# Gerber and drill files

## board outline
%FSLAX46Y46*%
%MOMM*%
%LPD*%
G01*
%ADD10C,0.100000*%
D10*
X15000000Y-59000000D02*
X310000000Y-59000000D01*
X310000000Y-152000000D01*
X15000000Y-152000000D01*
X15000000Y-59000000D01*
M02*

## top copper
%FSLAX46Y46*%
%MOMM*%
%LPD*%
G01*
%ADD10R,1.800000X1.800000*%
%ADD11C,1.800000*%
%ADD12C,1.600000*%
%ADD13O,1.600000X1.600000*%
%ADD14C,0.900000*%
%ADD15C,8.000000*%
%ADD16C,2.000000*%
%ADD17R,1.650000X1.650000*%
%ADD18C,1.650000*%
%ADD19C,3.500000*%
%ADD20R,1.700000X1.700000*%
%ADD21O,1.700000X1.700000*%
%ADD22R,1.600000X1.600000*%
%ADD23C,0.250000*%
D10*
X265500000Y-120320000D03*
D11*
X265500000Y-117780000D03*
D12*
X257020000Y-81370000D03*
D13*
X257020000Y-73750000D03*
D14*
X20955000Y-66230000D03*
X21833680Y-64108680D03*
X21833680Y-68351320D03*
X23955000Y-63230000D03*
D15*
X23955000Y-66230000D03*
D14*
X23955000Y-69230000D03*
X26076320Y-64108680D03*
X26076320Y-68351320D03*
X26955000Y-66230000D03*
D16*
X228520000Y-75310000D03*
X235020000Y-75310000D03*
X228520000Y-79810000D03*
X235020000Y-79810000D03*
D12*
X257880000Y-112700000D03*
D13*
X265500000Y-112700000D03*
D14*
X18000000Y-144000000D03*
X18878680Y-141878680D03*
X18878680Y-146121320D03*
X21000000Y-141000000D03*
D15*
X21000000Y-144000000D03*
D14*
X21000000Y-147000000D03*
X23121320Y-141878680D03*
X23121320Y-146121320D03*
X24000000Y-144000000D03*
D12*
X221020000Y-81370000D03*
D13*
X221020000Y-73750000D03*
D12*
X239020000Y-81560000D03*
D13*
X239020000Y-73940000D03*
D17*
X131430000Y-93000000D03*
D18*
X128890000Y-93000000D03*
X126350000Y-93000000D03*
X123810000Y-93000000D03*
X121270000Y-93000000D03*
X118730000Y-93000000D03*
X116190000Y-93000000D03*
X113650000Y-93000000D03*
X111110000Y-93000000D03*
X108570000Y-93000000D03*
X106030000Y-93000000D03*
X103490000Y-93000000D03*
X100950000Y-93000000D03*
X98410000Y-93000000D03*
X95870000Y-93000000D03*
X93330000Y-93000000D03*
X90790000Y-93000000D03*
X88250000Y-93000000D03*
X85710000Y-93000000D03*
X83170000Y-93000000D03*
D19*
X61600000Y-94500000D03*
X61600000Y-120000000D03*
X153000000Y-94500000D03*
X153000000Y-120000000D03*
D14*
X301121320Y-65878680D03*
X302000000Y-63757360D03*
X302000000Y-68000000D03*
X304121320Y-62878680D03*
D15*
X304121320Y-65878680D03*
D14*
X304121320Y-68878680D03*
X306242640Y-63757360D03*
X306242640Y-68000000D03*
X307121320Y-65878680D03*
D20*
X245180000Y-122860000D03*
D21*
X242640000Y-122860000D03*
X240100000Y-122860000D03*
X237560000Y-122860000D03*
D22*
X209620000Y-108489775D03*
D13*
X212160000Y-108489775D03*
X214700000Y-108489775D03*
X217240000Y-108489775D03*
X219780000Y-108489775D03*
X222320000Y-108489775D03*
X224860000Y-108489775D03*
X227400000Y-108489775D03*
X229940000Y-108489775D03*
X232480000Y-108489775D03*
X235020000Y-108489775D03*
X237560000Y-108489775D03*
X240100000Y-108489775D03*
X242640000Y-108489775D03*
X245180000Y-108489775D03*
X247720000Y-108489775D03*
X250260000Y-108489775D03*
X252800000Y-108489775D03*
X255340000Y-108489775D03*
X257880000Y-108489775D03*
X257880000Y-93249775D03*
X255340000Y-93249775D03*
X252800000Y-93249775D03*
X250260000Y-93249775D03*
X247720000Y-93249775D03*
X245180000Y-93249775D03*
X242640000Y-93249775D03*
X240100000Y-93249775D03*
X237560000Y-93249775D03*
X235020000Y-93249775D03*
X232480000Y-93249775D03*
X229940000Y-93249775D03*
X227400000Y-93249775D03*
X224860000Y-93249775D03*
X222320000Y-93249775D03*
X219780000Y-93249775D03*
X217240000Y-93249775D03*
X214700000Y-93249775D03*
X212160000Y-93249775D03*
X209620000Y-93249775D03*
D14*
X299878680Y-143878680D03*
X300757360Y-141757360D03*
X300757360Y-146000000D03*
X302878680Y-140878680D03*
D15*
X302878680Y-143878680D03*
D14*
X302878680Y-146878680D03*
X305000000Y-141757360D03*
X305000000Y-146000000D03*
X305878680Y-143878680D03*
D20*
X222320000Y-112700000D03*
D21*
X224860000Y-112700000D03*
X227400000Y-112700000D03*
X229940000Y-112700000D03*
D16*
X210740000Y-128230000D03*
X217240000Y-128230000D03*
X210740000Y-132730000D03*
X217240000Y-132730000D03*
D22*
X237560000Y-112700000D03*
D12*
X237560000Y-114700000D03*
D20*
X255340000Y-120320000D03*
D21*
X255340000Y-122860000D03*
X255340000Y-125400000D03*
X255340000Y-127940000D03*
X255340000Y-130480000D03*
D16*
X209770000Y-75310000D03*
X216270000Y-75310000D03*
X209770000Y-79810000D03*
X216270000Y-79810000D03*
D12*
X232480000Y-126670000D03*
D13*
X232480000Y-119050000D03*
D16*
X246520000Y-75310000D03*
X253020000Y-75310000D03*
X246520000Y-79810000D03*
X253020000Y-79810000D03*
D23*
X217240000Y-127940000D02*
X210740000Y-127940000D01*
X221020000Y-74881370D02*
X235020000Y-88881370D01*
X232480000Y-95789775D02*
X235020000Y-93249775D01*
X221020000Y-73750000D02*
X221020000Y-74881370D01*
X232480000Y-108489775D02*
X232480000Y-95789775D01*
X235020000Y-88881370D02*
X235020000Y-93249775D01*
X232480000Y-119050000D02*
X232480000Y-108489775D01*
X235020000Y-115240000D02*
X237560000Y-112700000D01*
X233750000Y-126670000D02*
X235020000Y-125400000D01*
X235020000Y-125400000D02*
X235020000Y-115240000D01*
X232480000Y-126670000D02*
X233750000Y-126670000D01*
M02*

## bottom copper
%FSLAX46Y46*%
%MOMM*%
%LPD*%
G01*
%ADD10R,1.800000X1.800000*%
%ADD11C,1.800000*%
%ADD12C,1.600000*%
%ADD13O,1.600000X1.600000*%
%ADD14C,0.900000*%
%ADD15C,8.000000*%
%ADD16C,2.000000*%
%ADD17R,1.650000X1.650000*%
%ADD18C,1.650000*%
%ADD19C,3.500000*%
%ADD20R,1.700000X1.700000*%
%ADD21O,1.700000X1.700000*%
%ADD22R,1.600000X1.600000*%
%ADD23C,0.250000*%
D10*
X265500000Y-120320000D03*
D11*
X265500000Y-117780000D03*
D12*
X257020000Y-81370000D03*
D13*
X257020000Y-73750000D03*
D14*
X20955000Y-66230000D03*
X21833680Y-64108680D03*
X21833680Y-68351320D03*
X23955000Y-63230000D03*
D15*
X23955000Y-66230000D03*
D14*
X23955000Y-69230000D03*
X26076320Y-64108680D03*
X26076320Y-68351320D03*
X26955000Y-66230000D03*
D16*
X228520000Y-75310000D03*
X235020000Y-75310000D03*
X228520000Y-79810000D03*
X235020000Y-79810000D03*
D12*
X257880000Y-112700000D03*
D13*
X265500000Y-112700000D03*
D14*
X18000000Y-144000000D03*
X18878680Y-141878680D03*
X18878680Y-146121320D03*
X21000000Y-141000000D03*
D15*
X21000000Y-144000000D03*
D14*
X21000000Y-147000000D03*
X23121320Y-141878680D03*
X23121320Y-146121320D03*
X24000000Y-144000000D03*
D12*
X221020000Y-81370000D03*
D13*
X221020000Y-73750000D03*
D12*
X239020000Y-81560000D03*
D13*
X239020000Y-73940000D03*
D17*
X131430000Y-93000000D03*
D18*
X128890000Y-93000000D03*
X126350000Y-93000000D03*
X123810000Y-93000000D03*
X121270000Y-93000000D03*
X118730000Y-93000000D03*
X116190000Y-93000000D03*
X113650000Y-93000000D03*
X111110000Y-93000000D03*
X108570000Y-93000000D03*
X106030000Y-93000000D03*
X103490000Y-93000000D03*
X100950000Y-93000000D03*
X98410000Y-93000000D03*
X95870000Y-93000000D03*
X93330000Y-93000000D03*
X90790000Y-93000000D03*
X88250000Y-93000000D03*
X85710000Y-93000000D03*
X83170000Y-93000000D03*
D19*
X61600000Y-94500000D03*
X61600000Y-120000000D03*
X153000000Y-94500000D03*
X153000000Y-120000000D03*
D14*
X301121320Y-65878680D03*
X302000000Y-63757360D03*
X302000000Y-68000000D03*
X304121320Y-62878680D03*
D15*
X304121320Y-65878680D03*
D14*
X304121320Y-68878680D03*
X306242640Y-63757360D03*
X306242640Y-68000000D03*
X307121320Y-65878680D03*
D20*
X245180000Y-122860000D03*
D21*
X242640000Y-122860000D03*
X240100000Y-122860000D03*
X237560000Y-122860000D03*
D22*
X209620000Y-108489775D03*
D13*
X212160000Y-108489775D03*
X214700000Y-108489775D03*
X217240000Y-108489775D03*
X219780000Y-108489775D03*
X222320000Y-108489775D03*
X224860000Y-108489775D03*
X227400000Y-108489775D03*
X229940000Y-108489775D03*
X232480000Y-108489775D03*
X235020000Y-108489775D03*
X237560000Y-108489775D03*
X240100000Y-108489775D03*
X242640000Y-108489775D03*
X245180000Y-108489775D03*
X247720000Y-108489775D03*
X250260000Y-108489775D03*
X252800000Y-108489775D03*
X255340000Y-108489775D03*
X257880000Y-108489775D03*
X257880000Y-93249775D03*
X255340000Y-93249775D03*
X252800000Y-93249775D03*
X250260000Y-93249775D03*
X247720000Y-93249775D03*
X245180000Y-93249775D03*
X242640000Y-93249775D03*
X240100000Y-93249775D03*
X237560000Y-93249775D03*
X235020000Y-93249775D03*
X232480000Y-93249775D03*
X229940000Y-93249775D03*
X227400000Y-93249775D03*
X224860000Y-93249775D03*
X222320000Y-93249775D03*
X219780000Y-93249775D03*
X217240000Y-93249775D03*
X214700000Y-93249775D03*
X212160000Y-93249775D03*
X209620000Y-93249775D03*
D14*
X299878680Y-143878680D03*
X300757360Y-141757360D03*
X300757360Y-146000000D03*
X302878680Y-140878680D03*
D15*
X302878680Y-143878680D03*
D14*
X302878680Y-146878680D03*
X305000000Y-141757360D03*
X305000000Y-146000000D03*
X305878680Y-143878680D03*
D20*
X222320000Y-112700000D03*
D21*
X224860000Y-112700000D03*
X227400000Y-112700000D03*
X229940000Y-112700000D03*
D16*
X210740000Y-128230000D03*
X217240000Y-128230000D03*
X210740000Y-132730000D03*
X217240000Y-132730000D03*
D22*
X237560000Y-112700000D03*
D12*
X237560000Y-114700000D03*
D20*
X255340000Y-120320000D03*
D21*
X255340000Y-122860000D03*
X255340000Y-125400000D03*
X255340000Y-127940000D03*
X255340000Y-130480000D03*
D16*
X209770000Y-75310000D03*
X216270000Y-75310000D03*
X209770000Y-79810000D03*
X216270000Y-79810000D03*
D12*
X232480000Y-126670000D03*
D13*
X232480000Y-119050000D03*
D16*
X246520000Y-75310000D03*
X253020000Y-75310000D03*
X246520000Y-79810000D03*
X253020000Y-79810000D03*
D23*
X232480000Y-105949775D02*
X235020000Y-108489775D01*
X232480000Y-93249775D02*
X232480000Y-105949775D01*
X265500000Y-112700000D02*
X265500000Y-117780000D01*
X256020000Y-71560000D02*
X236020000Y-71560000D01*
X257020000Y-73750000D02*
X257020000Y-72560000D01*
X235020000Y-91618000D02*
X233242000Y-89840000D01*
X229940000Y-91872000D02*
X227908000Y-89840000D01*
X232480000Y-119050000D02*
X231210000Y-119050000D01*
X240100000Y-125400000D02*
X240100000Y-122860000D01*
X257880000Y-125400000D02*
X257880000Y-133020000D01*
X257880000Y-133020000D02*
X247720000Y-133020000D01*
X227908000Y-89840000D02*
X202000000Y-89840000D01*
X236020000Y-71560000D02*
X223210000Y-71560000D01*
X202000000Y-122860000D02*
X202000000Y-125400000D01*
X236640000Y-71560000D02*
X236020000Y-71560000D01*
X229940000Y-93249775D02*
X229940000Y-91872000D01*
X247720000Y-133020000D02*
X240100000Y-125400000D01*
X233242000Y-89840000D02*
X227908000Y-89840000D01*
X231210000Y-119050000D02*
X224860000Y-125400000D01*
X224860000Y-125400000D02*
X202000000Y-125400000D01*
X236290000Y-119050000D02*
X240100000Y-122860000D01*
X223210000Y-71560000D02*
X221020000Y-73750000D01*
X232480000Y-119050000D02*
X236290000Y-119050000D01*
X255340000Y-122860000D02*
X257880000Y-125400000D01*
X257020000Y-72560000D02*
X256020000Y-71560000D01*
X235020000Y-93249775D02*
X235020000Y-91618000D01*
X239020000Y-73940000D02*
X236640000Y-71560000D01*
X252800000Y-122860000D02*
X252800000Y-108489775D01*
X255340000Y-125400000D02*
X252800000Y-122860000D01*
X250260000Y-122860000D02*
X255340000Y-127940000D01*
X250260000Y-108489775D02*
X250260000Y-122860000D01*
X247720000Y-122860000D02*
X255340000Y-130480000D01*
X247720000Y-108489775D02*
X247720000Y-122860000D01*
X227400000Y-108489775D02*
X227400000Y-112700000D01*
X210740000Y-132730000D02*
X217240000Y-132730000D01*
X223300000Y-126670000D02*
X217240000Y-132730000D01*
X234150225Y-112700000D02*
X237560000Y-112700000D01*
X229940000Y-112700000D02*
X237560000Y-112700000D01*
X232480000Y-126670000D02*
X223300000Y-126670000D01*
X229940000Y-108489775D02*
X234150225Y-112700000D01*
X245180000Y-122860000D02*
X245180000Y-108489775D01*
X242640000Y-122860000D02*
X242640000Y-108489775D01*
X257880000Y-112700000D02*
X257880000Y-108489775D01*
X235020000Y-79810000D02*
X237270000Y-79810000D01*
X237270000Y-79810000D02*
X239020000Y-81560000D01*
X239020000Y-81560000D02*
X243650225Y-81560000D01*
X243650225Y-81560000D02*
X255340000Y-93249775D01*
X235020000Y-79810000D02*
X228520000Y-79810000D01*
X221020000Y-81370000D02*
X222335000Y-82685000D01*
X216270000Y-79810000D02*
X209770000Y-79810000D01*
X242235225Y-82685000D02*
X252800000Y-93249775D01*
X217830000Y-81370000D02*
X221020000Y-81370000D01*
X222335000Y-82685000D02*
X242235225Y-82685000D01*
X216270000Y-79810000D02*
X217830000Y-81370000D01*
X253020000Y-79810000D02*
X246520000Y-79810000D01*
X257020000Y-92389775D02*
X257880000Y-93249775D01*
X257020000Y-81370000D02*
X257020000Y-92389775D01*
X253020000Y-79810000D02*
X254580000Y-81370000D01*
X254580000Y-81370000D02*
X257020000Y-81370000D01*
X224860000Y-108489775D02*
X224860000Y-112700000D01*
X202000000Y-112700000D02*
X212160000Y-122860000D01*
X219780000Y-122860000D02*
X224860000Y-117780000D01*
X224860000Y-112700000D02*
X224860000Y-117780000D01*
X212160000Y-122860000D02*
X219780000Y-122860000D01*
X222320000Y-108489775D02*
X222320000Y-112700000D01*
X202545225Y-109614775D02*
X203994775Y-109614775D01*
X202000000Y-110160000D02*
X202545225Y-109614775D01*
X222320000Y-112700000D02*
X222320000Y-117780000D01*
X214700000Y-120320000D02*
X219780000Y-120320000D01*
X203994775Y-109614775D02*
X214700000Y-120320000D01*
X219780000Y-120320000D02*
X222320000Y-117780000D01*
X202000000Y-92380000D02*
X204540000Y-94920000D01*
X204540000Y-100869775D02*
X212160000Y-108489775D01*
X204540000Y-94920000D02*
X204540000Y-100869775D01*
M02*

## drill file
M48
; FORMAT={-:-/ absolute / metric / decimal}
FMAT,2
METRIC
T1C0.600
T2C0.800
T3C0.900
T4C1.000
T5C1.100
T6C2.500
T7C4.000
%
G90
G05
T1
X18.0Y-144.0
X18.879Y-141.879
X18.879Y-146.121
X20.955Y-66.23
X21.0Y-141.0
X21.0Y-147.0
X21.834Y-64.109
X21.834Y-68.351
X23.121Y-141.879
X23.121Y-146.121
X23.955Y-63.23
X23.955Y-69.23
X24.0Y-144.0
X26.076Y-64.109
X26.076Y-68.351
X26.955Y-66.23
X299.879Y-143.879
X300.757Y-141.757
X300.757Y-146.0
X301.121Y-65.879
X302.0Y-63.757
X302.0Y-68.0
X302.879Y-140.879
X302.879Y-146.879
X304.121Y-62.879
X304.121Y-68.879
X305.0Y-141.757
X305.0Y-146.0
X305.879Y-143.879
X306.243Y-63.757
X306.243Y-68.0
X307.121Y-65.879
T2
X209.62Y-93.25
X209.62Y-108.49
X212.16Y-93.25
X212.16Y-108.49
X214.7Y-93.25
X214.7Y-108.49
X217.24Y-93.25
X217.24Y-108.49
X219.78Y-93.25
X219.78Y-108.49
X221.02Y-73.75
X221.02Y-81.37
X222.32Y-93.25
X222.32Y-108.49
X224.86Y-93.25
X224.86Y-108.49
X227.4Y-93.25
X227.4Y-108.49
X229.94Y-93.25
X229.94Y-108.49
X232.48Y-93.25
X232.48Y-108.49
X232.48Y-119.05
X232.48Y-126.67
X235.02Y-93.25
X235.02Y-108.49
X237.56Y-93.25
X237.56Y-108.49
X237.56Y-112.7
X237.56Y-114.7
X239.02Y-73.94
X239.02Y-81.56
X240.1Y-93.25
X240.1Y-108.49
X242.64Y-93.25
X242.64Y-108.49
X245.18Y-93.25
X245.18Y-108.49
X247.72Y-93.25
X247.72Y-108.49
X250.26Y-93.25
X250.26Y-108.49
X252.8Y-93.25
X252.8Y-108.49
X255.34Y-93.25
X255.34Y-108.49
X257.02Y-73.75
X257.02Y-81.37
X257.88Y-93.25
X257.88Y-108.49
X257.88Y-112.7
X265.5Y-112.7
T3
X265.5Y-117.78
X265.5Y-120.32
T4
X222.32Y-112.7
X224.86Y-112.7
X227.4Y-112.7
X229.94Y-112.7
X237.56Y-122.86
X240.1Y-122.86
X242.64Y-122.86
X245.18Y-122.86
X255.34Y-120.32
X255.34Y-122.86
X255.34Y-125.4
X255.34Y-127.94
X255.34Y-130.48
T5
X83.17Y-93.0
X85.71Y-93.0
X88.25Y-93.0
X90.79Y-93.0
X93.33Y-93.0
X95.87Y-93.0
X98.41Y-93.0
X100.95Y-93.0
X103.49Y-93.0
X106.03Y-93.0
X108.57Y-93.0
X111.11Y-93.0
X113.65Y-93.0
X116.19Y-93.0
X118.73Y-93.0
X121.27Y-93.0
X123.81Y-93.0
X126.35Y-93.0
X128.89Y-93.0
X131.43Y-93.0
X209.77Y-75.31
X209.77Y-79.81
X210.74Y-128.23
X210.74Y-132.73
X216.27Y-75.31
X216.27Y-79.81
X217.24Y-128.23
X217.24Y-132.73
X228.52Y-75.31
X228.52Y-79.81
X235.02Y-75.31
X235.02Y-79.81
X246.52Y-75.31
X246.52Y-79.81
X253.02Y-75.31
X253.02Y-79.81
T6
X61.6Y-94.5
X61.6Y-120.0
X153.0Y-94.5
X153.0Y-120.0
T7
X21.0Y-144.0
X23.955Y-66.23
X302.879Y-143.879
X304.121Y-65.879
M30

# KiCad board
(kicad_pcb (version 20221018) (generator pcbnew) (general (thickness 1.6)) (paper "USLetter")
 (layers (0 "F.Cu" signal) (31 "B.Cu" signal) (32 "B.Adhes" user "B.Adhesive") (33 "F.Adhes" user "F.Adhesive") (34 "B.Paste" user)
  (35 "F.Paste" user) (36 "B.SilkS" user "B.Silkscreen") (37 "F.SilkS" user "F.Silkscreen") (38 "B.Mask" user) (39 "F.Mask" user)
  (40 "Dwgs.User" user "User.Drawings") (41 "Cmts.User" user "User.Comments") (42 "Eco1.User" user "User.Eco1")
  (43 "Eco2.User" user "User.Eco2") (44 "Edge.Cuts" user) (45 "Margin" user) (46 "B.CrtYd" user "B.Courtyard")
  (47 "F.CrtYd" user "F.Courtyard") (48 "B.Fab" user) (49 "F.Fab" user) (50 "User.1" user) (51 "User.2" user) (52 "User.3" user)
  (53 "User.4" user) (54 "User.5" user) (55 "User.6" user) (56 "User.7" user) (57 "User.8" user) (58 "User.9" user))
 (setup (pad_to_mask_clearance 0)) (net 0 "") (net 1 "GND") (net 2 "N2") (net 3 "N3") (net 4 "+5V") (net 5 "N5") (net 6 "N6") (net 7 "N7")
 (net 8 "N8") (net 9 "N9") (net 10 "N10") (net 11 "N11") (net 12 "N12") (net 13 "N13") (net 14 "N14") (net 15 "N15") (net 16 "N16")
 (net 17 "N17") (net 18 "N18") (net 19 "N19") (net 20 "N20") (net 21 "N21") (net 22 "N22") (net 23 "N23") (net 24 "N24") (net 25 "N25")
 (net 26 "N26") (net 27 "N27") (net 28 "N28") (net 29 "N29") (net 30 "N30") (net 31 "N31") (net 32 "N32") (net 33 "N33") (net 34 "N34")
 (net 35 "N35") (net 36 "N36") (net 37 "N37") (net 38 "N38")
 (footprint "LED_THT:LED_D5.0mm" (layer "F.Cu") (at 265.5 120.32 90)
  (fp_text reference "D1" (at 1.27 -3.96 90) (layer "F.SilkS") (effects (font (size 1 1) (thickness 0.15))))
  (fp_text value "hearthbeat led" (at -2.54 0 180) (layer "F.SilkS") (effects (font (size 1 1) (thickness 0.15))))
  (pad "1" thru_hole rect (at 0 0 90) (size 1.8 1.8) (drill 0.9) (layers "*.Cu" "*.Mask") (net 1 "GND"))
  (pad "2" thru_hole circle (at 2.54 0 90) (size 1.8 1.8) (drill 0.9) (layers "*.Cu" "*.Mask") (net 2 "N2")))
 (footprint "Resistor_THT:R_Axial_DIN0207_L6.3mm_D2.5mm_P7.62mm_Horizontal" (layer "F.Cu") (at 257.02 81.37 90)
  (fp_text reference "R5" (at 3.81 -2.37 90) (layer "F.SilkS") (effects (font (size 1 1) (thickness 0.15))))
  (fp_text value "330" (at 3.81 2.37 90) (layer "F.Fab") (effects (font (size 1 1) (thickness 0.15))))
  (pad "1" thru_hole circle (at 0 0 90) (size 1.6 1.6) (drill 0.8) (layers "*.Cu" "*.Mask") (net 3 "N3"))
  (pad "2" thru_hole oval (at 7.62 0 90) (size 1.6 1.6) (drill 0.8) (layers "*.Cu" "*.Mask") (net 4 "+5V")))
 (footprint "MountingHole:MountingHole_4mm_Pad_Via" (layer "F.Cu") (at 23.955 66.23)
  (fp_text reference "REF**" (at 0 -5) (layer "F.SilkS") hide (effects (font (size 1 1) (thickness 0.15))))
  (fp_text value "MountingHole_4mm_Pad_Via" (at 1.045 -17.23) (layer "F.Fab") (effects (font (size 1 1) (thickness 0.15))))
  (pad "1" thru_hole circle (at -3 0) (size 0.9 0.9) (drill 0.6) (layers "*.Cu" "*.Mask"))
  (pad "1" thru_hole circle (at -2.12132 -2.12132) (size 0.9 0.9) (drill 0.6) (layers "*.Cu" "*.Mask"))
  (pad "1" thru_hole circle (at -2.12132 2.12132) (size 0.9 0.9) (drill 0.6) (layers "*.Cu" "*.Mask"))
  (pad "1" thru_hole circle (at 0 -3) (size 0.9 0.9) (drill 0.6) (layers "*.Cu" "*.Mask"))
  (pad "1" thru_hole circle (at 0 0) (size 8 8) (drill 4) (layers "*.Cu" "*.Mask"))
  (pad "1" thru_hole circle (at 0 3) (size 0.9 0.9) (drill 0.6) (layers "*.Cu" "*.Mask"))
  (pad "1" thru_hole circle (at 2.12132 -2.12132) (size 0.9 0.9) (drill 0.6) (layers "*.Cu" "*.Mask"))
  (pad "1" thru_hole circle (at 2.12132 2.12132) (size 0.9 0.9) (drill 0.6) (layers "*.Cu" "*.Mask"))
  (pad "1" thru_hole circle (at 3 0) (size 0.9 0.9) (drill 0.6) (layers "*.Cu" "*.Mask")))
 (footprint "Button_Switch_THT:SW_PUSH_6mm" (layer "F.Cu") (at 228.52 75.31)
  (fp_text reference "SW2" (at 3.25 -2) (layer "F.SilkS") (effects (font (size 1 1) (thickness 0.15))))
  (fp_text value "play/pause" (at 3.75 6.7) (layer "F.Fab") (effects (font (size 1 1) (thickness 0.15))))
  (pad "1" thru_hole circle (at 0 0 90) (size 2 2) (drill 1.1) (layers "*.Cu" "*.Mask") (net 1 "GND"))
  (pad "1" thru_hole circle (at 6.5 0 90) (size 2 2) (drill 1.1) (layers "*.Cu" "*.Mask") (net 1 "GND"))
  (pad "2" thru_hole circle (at 0 4.5 90) (size 2 2) (drill 1.1) (layers "*.Cu" "*.Mask") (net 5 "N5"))
  (pad "2" thru_hole circle (at 6.5 4.5 90) (size 2 2) (drill 1.1) (layers "*.Cu" "*.Mask") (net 5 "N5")))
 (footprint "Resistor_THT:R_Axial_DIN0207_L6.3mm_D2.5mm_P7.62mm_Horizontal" (layer "F.Cu") (at 257.88 112.7)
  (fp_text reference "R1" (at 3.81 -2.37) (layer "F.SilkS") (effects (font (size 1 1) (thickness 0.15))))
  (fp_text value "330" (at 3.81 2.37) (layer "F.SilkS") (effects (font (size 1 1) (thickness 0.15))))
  (pad "1" thru_hole circle (at 0 0) (size 1.6 1.6) (drill 0.8) (layers "*.Cu" "*.Mask") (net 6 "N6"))
  (pad "2" thru_hole oval (at 7.62 0) (size 1.6 1.6) (drill 0.8) (layers "*.Cu" "*.Mask") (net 2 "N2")))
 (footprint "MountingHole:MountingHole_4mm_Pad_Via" (layer "F.Cu") (at 21 144)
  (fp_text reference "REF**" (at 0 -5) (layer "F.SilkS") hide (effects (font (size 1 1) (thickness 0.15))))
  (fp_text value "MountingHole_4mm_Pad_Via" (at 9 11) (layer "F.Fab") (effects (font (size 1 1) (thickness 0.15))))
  (pad "1" thru_hole circle (at -3 0) (size 0.9 0.9) (drill 0.6) (layers "*.Cu" "*.Mask"))
  (pad "1" thru_hole circle (at -2.12132 -2.12132) (size 0.9 0.9) (drill 0.6) (layers "*.Cu" "*.Mask"))
  (pad "1" thru_hole circle (at -2.12132 2.12132) (size 0.9 0.9) (drill 0.6) (layers "*.Cu" "*.Mask"))
  (pad "1" thru_hole circle (at 0 -3) (size 0.9 0.9) (drill 0.6) (layers "*.Cu" "*.Mask"))
  (pad "1" thru_hole circle (at 0 0) (size 8 8) (drill 4) (layers "*.Cu" "*.Mask"))
  (pad "1" thru_hole circle (at 0 3) (size 0.9 0.9) (drill 0.6) (layers "*.Cu" "*.Mask"))
  (pad "1" thru_hole circle (at 2.12132 -2.12132) (size 0.9 0.9) (drill 0.6) (layers "*.Cu" "*.Mask"))
  (pad "1" thru_hole circle (at 2.12132 2.12132) (size 0.9 0.9) (drill 0.6) (layers "*.Cu" "*.Mask"))
  (pad "1" thru_hole circle (at 3 0) (size 0.9 0.9) (drill 0.6) (layers "*.Cu" "*.Mask")))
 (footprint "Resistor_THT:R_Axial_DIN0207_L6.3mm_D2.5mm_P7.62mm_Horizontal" (layer "F.Cu") (at 221.02 81.37 90)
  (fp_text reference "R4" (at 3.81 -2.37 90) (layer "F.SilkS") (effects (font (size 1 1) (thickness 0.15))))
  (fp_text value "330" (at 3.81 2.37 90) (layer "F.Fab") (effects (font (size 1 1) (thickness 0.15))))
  (pad "1" thru_hole circle (at 0 0 90) (size 1.6 1.6) (drill 0.8) (layers "*.Cu" "*.Mask") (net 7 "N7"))
  (pad "2" thru_hole oval (at 7.62 0 90) (size 1.6 1.6) (drill 0.8) (layers "*.Cu" "*.Mask") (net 4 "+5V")))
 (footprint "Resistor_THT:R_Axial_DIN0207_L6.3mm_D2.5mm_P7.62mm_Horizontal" (layer "F.Cu") (at 239.02 81.56 90)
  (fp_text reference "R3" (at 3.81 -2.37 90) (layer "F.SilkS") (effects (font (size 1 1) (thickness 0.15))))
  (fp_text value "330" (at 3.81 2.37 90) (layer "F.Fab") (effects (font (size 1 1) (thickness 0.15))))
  (pad "1" thru_hole circle (at 0 0 90) (size 1.6 1.6) (drill 0.8) (layers "*.Cu" "*.Mask") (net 5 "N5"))
  (pad "2" thru_hole oval (at 7.62 0 90) (size 1.6 1.6) (drill 0.8) (layers "*.Cu" "*.Mask") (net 4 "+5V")))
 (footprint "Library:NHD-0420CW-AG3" (layer "F.Cu") (at 107.3 107.25)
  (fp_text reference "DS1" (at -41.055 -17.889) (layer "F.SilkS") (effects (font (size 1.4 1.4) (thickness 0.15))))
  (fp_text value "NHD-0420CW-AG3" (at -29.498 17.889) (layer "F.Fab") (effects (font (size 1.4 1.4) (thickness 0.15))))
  (pad "1" thru_hole rect (at 24.13 -14.25) (size 1.65 1.65) (drill 1.1) (layers "*.Cu" "*.Mask") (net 1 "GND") (solder_mask_margin 0.102))
  (pad "2" thru_hole circle (at 21.59 -14.25) (size 1.65 1.65) (drill 1.1) (layers "*.Cu" "*.Mask") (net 4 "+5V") (solder_mask_margin 0.102))
  (pad "3" thru_hole circle (at 19.05 -14.25) (size 1.65 1.65) (drill 1.1) (layers "*.Cu" "*.Mask") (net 4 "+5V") (solder_mask_margin 0.102))
  (pad "4" thru_hole circle (at 16.51 -14.25) (size 1.65 1.65) (drill 1.1) (layers "*.Cu" "*.Mask") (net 1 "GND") (solder_mask_margin 0.102))
  (pad "5" thru_hole circle (at 13.97 -14.25) (size 1.65 1.65) (drill 1.1) (layers "*.Cu" "*.Mask") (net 1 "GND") (solder_mask_margin 0.102))
  (pad "6" thru_hole circle (at 11.43 -14.25) (size 1.65 1.65) (drill 1.1) (layers "*.Cu" "*.Mask") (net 1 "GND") (solder_mask_margin 0.102))
  (pad "7" thru_hole circle (at 8.89 -14.25) (size 1.65 1.65) (drill 1.1) (layers "*.Cu" "*.Mask") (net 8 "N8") (solder_mask_margin 0.102))
  (pad "8" thru_hole circle (at 6.35 -14.25) (size 1.65 1.65) (drill 1.1) (layers "*.Cu" "*.Mask") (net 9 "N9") (solder_mask_margin 0.102))
  (pad "9" thru_hole circle (at 3.81 -14.25) (size 1.65 1.65) (drill 1.1) (layers "*.Cu" "*.Mask") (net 1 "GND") (solder_mask_margin 0.102))
  (pad "10" thru_hole circle (at 1.27 -14.25) (size 1.65 1.65) (drill 1.1) (layers "*.Cu" "*.Mask") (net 1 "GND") (solder_mask_margin 0.102))
  (pad "11" thru_hole circle (at -1.27 -14.25) (size 1.65 1.65) (drill 1.1) (layers "*.Cu" "*.Mask") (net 1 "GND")
   (solder_mask_margin 0.102))
  (pad "12" thru_hole circle (at -3.81 -14.25) (size 1.65 1.65) (drill 1.1) (layers "*.Cu" "*.Mask") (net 1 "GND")
   (solder_mask_margin 0.102))
  (pad "13" thru_hole circle (at -6.35 -14.25) (size 1.65 1.65) (drill 1.1) (layers "*.Cu" "*.Mask") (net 1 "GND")
   (solder_mask_margin 0.102))
  (pad "14" thru_hole circle (at -8.89 -14.25) (size 1.65 1.65) (drill 1.1) (layers "*.Cu" "*.Mask") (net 1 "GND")
   (solder_mask_margin 0.102))
  (pad "15" thru_hole circle (at -11.43 -14.25) (size 1.65 1.65) (drill 1.1) (layers "*.Cu" "*.Mask") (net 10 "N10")
   (solder_mask_margin 0.102))
  (pad "16" thru_hole circle (at -13.97 -14.25) (size 1.65 1.65) (drill 1.1) (layers "*.Cu" "*.Mask") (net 4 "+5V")
   (solder_mask_margin 0.102))
  (pad "17" thru_hole circle (at -16.51 -14.25) (size 1.65 1.65) (drill 1.1) (layers "*.Cu" "*.Mask") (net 1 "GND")
   (solder_mask_margin 0.102))
  (pad "18" thru_hole circle (at -19.05 -14.25) (size 1.65 1.65) (drill 1.1) (layers "*.Cu" "*.Mask") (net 1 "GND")
   (solder_mask_margin 0.102))
  (pad "19" thru_hole circle (at -21.59 -14.25) (size 1.65 1.65) (drill 1.1) (layers "*.Cu" "*.Mask") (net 1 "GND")
   (solder_mask_margin 0.102))
  (pad "20" thru_hole circle (at -24.13 -14.25) (size 1.65 1.65) (drill 1.1) (layers "*.Cu" "*.Mask") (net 1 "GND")
   (solder_mask_margin 0.102))
  (pad "P1" thru_hole circle (at -45.7 -12.75) (size 3.5 3.5) (drill 2.5) (layers "*.Cu" "*.Mask") (solder_mask_margin 0.102))
  (pad "P2" thru_hole circle (at -45.7 12.75) (size 3.5 3.5) (drill 2.5) (layers "*.Cu" "*.Mask") (solder_mask_margin 0.102))
  (pad "P3" thru_hole circle (at 45.7 -12.75) (size 3.5 3.5) (drill 2.5) (layers "*.Cu" "*.Mask") (solder_mask_margin 0.102))
  (pad "P4" thru_hole circle (at 45.7 12.75) (size 3.5 3.5) (drill 2.5) (layers "*.Cu" "*.Mask") (solder_mask_margin 0.102)))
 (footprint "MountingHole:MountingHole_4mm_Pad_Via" (layer "F.Cu") (at 304.12132 65.87868)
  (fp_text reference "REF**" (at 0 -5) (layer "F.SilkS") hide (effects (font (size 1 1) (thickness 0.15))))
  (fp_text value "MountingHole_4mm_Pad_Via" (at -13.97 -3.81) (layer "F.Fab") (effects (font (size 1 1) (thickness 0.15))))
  (pad "1" thru_hole circle (at -3 0) (size 0.9 0.9) (drill 0.6) (layers "*.Cu" "*.Mask"))
  (pad "1" thru_hole circle (at -2.12132 -2.12132) (size 0.9 0.9) (drill 0.6) (layers "*.Cu" "*.Mask"))
  (pad "1" thru_hole circle (at -2.12132 2.12132) (size 0.9 0.9) (drill 0.6) (layers "*.Cu" "*.Mask"))
  (pad "1" thru_hole circle (at 0 -3) (size 0.9 0.9) (drill 0.6) (layers "*.Cu" "*.Mask"))
  (pad "1" thru_hole circle (at 0 0) (size 8 8) (drill 4) (layers "*.Cu" "*.Mask"))
  (pad "1" thru_hole circle (at 0 3) (size 0.9 0.9) (drill 0.6) (layers "*.Cu" "*.Mask"))
  (pad "1" thru_hole circle (at 2.12132 -2.12132) (size 0.9 0.9) (drill 0.6) (layers "*.Cu" "*.Mask"))
  (pad "1" thru_hole circle (at 2.12132 2.12132) (size 0.9 0.9) (drill 0.6) (layers "*.Cu" "*.Mask"))
  (pad "1" thru_hole circle (at 3 0) (size 0.9 0.9) (drill 0.6) (layers "*.Cu" "*.Mask")))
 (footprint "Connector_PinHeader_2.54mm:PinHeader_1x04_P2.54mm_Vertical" (layer "F.Cu") (at 245.18 122.86 -90)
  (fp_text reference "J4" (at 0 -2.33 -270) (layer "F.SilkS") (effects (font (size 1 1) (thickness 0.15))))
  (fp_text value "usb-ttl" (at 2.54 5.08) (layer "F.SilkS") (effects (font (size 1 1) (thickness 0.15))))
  (pad "1" thru_hole rect (at 0 0 270) (size 1.7 1.7) (drill 1) (layers "*.Cu" "*.Mask") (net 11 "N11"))
  (pad "2" thru_hole oval (at 0 2.54 270) (size 1.7 1.7) (drill 1) (layers "*.Cu" "*.Mask") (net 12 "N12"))
  (pad "3" thru_hole oval (at 0 5.08 270) (size 1.7 1.7) (drill 1) (layers "*.Cu" "*.Mask") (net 4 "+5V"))
  (pad "4" thru_hole oval (at 0 7.62 270) (size 1.7 1.7) (drill 1) (layers "*.Cu" "*.Mask") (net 1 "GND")))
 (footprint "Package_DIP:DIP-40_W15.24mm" (layer "F.Cu") (at 209.62 108.489775 90)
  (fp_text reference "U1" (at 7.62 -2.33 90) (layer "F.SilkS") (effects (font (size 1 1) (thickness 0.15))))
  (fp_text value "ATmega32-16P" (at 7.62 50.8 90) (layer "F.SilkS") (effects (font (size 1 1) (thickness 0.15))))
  (pad "1" thru_hole rect (at 0 0 90) (size 1.6 1.6) (drill 0.8) (layers "*.Cu" "*.Mask") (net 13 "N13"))
  (pad "2" thru_hole oval (at 0 2.54 90) (size 1.6 1.6) (drill 0.8) (layers "*.Cu" "*.Mask") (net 10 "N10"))
  (pad "3" thru_hole oval (at 0 5.08 90) (size 1.6 1.6) (drill 0.8) (layers "*.Cu" "*.Mask") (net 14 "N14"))
  (pad "4" thru_hole oval (at 0 7.62 90) (size 1.6 1.6) (drill 0.8) (layers "*.Cu" "*.Mask") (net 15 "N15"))
  (pad "5" thru_hole oval (at 0 10.16 90) (size 1.6 1.6) (drill 0.8) (layers "*.Cu" "*.Mask") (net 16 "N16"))
  (pad "6" thru_hole oval (at 0 12.7 90) (size 1.6 1.6) (drill 0.8) (layers "*.Cu" "*.Mask") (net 9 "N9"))
  (pad "7" thru_hole oval (at 0 15.24 90) (size 1.6 1.6) (drill 0.8) (layers "*.Cu" "*.Mask") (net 8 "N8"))
  (pad "8" thru_hole oval (at 0 17.78 90) (size 1.6 1.6) (drill 0.8) (layers "*.Cu" "*.Mask") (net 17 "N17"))
  (pad "9" thru_hole oval (at 0 20.32 90) (size 1.6 1.6) (drill 0.8) (layers "*.Cu" "*.Mask") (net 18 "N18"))
  (pad "10" thru_hole oval (at 0 22.86 90) (size 1.6 1.6) (drill 0.8) (layers "*.Cu" "*.Mask") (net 4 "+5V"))
  (pad "11" thru_hole oval (at 0 25.4 90) (size 1.6 1.6) (drill 0.8) (layers "*.Cu" "*.Mask") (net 1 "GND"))
  (pad "12" thru_hole oval (at 0 27.94 90) (size 1.6 1.6) (drill 0.8) (layers "*.Cu" "*.Mask") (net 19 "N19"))
  (pad "13" thru_hole oval (at 0 30.48 90) (size 1.6 1.6) (drill 0.8) (layers "*.Cu" "*.Mask") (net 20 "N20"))
  (pad "14" thru_hole oval (at 0 33.02 90) (size 1.6 1.6) (drill 0.8) (layers "*.Cu" "*.Mask") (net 12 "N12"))
  (pad "15" thru_hole oval (at 0 35.56 90) (size 1.6 1.6) (drill 0.8) (layers "*.Cu" "*.Mask") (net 11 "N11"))
  (pad "16" thru_hole oval (at 0 38.1 90) (size 1.6 1.6) (drill 0.8) (layers "*.Cu" "*.Mask") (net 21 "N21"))
  (pad "17" thru_hole oval (at 0 40.64 90) (size 1.6 1.6) (drill 0.8) (layers "*.Cu" "*.Mask") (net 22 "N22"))
  (pad "18" thru_hole oval (at 0 43.18 90) (size 1.6 1.6) (drill 0.8) (layers "*.Cu" "*.Mask") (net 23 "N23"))
  (pad "19" thru_hole oval (at 0 45.72 90) (size 1.6 1.6) (drill 0.8) (layers "*.Cu" "*.Mask") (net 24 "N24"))
  (pad "20" thru_hole oval (at 0 48.26 90) (size 1.6 1.6) (drill 0.8) (layers "*.Cu" "*.Mask") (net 6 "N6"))
  (pad "21" thru_hole oval (at 15.24 48.26 90) (size 1.6 1.6) (drill 0.8) (layers "*.Cu" "*.Mask") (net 3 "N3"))
  (pad "22" thru_hole oval (at 15.24 45.72 90) (size 1.6 1.6) (drill 0.8) (layers "*.Cu" "*.Mask") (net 5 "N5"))
  (pad "23" thru_hole oval (at 15.24 43.18 90) (size 1.6 1.6) (drill 0.8) (layers "*.Cu" "*.Mask") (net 7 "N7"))
  (pad "24" thru_hole oval (at 15.24 40.64 90) (size 1.6 1.6) (drill 0.8) (layers "*.Cu" "*.Mask") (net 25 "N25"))
  (pad "25" thru_hole oval (at 15.24 38.1 90) (size 1.6 1.6) (drill 0.8) (layers "*.Cu" "*.Mask") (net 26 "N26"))
  (pad "26" thru_hole oval (at 15.24 35.56 90) (size 1.6 1.6) (drill 0.8) (layers "*.Cu" "*.Mask") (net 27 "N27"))
  (pad "27" thru_hole oval (at 15.24 33.02 90) (size 1.6 1.6) (drill 0.8) (layers "*.Cu" "*.Mask") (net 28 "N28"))
  (pad "28" thru_hole oval (at 15.24 30.48 90) (size 1.6 1.6) (drill 0.8) (layers "*.Cu" "*.Mask") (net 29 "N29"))
  (pad "29" thru_hole oval (at 15.24 27.94 90) (size 1.6 1.6) (drill 0.8) (layers "*.Cu" "*.Mask") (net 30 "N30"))
  (pad "30" thru_hole oval (at 15.24 25.4 90) (size 1.6 1.6) (drill 0.8) (layers "*.Cu" "*.Mask") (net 4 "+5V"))
  (pad "31" thru_hole oval (at 15.24 22.86 90) (size 1.6 1.6) (drill 0.8) (layers "*.Cu" "*.Mask") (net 1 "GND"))
  (pad "32" thru_hole oval (at 15.24 20.32 90) (size 1.6 1.6) (drill 0.8) (layers "*.Cu" "*.Mask") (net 4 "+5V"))
  (pad "33" thru_hole oval (at 15.24 17.78 90) (size 1.6 1.6) (drill 0.8) (layers "*.Cu" "*.Mask") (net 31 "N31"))
  (pad "34" thru_hole oval (at 15.24 15.24 90) (size 1.6 1.6) (drill 0.8) (layers "*.Cu" "*.Mask") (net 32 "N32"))
  (pad "35" thru_hole oval (at 15.24 12.7 90) (size 1.6 1.6) (drill 0.8) (layers "*.Cu" "*.Mask") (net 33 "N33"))
  (pad "36" thru_hole oval (at 15.24 10.16 90) (size 1.6 1.6) (drill 0.8) (layers "*.Cu" "*.Mask") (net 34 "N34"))
  (pad "37" thru_hole oval (at 15.24 7.62 90) (size 1.6 1.6) (drill 0.8) (layers "*.Cu" "*.Mask") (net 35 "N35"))
  (pad "38" thru_hole oval (at 15.24 5.08 90) (size 1.6 1.6) (drill 0.8) (layers "*.Cu" "*.Mask") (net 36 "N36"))
  (pad "39" thru_hole oval (at 15.24 2.54 90) (size 1.6 1.6) (drill 0.8) (layers "*.Cu" "*.Mask") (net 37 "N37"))
  (pad "40" thru_hole oval (at 15.24 0 90) (size 1.6 1.6) (drill 0.8) (layers "*.Cu" "*.Mask") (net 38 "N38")))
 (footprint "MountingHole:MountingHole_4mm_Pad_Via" (layer "F.Cu") (at 302.87868 143.87868)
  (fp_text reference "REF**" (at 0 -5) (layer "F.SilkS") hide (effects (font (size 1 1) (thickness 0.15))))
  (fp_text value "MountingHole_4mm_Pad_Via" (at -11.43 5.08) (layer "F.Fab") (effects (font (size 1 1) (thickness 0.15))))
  (pad "1" thru_hole circle (at -3 0) (size 0.9 0.9) (drill 0.6) (layers "*.Cu" "*.Mask"))
  (pad "1" thru_hole circle (at -2.12132 -2.12132) (size 0.9 0.9) (drill 0.6) (layers "*.Cu" "*.Mask"))
  (pad "1" thru_hole circle (at -2.12132 2.12132) (size 0.9 0.9) (drill 0.6) (layers "*.Cu" "*.Mask"))
  (pad "1" thru_hole circle (at 0 -3) (size 0.9 0.9) (drill 0.6) (layers "*.Cu" "*.Mask"))
  (pad "1" thru_hole circle (at 0 0) (size 8 8) (drill 4) (layers "*.Cu" "*.Mask"))
  (pad "1" thru_hole circle (at 0 3) (size 0.9 0.9) (drill 0.6) (layers "*.Cu" "*.Mask"))
  (pad "1" thru_hole circle (at 2.12132 -2.12132) (size 0.9 0.9) (drill 0.6) (layers "*.Cu" "*.Mask"))
  (pad "1" thru_hole circle (at 2.12132 2.12132) (size 0.9 0.9) (drill 0.6) (layers "*.Cu" "*.Mask"))
  (pad "1" thru_hole circle (at 3 0) (size 0.9 0.9) (drill 0.6) (layers "*.Cu" "*.Mask")))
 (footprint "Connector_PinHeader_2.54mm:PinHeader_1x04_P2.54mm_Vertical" (layer "F.Cu") (at 222.32 112.7 90)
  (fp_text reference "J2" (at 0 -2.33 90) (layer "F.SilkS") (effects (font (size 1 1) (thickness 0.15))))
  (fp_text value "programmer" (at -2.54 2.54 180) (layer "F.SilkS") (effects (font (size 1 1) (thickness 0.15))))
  (pad "1" thru_hole rect (at 0 0 90) (size 1.7 1.7) (drill 1) (layers "*.Cu" "*.Mask") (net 9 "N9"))
  (pad "2" thru_hole oval (at 0 2.54 90) (size 1.7 1.7) (drill 1) (layers "*.Cu" "*.Mask") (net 8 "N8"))
  (pad "3" thru_hole oval (at 0 5.08 90) (size 1.7 1.7) (drill 1) (layers "*.Cu" "*.Mask") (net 17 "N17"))
  (pad "4" thru_hole oval (at 0 7.62 90) (size 1.7 1.7) (drill 1) (layers "*.Cu" "*.Mask") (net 18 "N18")))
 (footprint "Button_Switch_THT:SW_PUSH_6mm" (layer "F.Cu") (at 210.74 128.23)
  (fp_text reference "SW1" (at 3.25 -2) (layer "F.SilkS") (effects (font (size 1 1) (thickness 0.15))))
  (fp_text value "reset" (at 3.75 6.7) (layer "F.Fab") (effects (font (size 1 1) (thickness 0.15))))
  (pad "1" thru_hole circle (at 0 0 90) (size 2 2) (drill 1.1) (layers "*.Cu" "*.Mask") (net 1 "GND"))
  (pad "1" thru_hole circle (at 6.5 0 90) (size 2 2) (drill 1.1) (layers "*.Cu" "*.Mask") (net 1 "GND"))
  (pad "2" thru_hole circle (at 0 4.5 90) (size 2 2) (drill 1.1) (layers "*.Cu" "*.Mask") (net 18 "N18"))
  (pad "2" thru_hole circle (at 6.5 4.5 90) (size 2 2) (drill 1.1) (layers "*.Cu" "*.Mask") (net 18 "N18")))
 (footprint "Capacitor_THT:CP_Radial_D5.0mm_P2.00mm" (layer "F.Cu") (at 237.56 112.7 -90)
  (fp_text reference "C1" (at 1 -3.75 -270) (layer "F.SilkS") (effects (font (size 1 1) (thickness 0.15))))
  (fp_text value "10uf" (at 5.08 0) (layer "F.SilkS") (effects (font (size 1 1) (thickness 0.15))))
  (pad "1" thru_hole rect (at 0 0 270) (size 1.6 1.6) (drill 0.8) (layers "*.Cu" "*.Mask") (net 18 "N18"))
  (pad "2" thru_hole circle (at 2 0 270) (size 1.6 1.6) (drill 0.8) (layers "*.Cu" "*.Mask") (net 1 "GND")))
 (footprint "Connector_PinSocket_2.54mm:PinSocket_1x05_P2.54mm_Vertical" (layer "F.Cu") (at 255.34 120.32)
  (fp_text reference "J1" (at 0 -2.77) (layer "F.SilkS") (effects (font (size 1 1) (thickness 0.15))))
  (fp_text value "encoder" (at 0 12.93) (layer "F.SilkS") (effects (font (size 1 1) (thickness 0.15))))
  (pad "1" thru_hole rect (at 0 0) (size 1.7 1.7) (drill 1) (layers "*.Cu" "*.Mask") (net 1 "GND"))
  (pad "2" thru_hole oval (at 0 2.54) (size 1.7 1.7) (drill 1) (layers "*.Cu" "*.Mask") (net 4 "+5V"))
  (pad "3" thru_hole oval (at 0 5.08) (size 1.7 1.7) (drill 1) (layers "*.Cu" "*.Mask") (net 23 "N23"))
  (pad "4" thru_hole oval (at 0 7.62) (size 1.7 1.7) (drill 1) (layers "*.Cu" "*.Mask") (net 22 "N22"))
  (pad "5" thru_hole oval (at 0 10.16) (size 1.7 1.7) (drill 1) (layers "*.Cu" "*.Mask") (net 21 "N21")))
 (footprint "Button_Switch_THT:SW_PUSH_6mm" (layer "F.Cu") (at 209.77 75.31)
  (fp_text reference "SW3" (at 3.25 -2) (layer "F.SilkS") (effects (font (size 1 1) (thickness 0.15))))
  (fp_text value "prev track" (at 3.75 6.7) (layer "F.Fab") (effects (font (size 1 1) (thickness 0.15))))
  (pad "1" thru_hole circle (at 0 0 90) (size 2 2) (drill 1.1) (layers "*.Cu" "*.Mask") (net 1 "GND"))
  (pad "1" thru_hole circle (at 6.5 0 90) (size 2 2) (drill 1.1) (layers "*.Cu" "*.Mask") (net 1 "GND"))
  (pad "2" thru_hole circle (at 0 4.5 90) (size 2 2) (drill 1.1) (layers "*.Cu" "*.Mask") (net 7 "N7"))
  (pad "2" thru_hole circle (at 6.5 4.5 90) (size 2 2) (drill 1.1) (layers "*.Cu" "*.Mask") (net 7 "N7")))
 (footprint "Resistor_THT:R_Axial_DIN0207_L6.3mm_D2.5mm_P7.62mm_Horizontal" (layer "F.Cu") (at 232.48 126.67 90)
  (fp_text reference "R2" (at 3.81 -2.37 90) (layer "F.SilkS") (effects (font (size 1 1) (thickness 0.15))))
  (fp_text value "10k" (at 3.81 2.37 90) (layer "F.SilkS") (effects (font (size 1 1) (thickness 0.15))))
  (pad "1" thru_hole circle (at 0 0 90) (size 1.6 1.6) (drill 0.8) (layers "*.Cu" "*.Mask") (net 18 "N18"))
  (pad "2" thru_hole oval (at 7.62 0 90) (size 1.6 1.6) (drill 0.8) (layers "*.Cu" "*.Mask") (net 4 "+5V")))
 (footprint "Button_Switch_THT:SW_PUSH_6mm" (layer "F.Cu") (at 246.52 75.31)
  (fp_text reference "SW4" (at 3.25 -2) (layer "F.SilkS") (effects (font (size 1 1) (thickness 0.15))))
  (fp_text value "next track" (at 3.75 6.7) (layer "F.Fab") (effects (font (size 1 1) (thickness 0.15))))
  (pad "1" thru_hole circle (at 0 0 90) (size 2 2) (drill 1.1) (layers "*.Cu" "*.Mask") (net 1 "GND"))
  (pad "1" thru_hole circle (at 6.5 0 90) (size 2 2) (drill 1.1) (layers "*.Cu" "*.Mask") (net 1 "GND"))
  (pad "2" thru_hole circle (at 0 4.5 90) (size 2 2) (drill 1.1) (layers "*.Cu" "*.Mask") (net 3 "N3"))
  (pad "2" thru_hole circle (at 6.5 4.5 90) (size 2 2) (drill 1.1) (layers "*.Cu" "*.Mask") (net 3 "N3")))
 (gr_rect (start 15 59) (end 310 152) (stroke (width 0.1) (type default)) (fill none) (layer "Edge.Cuts"))
 (segment (start 217.24 127.94) (end 210.74 127.94) (width 0.25) (layer "F.Cu") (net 1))
 (segment (start 232.48 105.949775) (end 235.02 108.489775) (width 0.25) (layer "B.Cu") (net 1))
 (segment (start 232.48 93.249775) (end 232.48 105.949775) (width 0.25) (layer "B.Cu") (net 1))
 (segment (start 265.5 112.7) (end 265.5 117.78) (width 0.25) (layer "B.Cu") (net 2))
 (segment (start 221.02 74.88137) (end 235.02 88.88137) (width 0.25) (layer "F.Cu") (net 4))
 (segment (start 232.48 95.789775) (end 235.02 93.249775) (width 0.25) (layer "F.Cu") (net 4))
 (segment (start 221.02 73.75) (end 221.02 74.88137) (width 0.25) (layer "F.Cu") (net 4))
 (segment (start 232.48 108.489775) (end 232.48 95.789775) (width 0.25) (layer "F.Cu") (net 4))
 (segment (start 235.02 88.88137) (end 235.02 93.249775) (width 0.25) (layer "F.Cu") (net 4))
 (segment (start 232.48 119.05) (end 232.48 108.489775) (width 0.25) (layer "F.Cu") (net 4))
 (segment (start 256.02 71.56) (end 236.02 71.56) (width 0.25) (layer "B.Cu") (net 4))
 (segment (start 257.02 73.75) (end 257.02 72.56) (width 0.25) (layer "B.Cu") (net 4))
 (segment (start 235.02 91.618) (end 233.242 89.84) (width 0.25) (layer "B.Cu") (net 4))
 (segment (start 229.94 91.872) (end 227.908 89.84) (width 0.25) (layer "B.Cu") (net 4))
 (segment (start 232.48 119.05) (end 231.21 119.05) (width 0.25) (layer "B.Cu") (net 4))
 (segment (start 240.1 125.4) (end 240.1 122.86) (width 0.25) (layer "B.Cu") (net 4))
 (segment (start 257.88 125.4) (end 257.88 133.02) (width 0.25) (layer "B.Cu") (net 4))
 (segment (start 257.88 133.02) (end 247.72 133.02) (width 0.25) (layer "B.Cu") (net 4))
 (segment (start 227.908 89.84) (end 202 89.84) (width 0.25) (layer "B.Cu") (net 4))
 (segment (start 236.02 71.56) (end 223.21 71.56) (width 0.25) (layer "B.Cu") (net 4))
 (segment (start 202 122.86) (end 202 125.4) (width 0.25) (layer "B.Cu") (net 4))
 (segment (start 236.64 71.56) (end 236.02 71.56) (width 0.25) (layer "B.Cu") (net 4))
 (segment (start 229.94 93.249775) (end 229.94 91.872) (width 0.25) (layer "B.Cu") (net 4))
 (segment (start 247.72 133.02) (end 240.1 125.4) (width 0.25) (layer "B.Cu") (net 4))
 (segment (start 233.242 89.84) (end 227.908 89.84) (width 0.25) (layer "B.Cu") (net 4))
 (segment (start 231.21 119.05) (end 224.86 125.4) (width 0.25) (layer "B.Cu") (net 4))
 (segment (start 224.86 125.4) (end 202 125.4) (width 0.25) (layer "B.Cu") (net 4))
 (segment (start 236.29 119.05) (end 240.1 122.86) (width 0.25) (layer "B.Cu") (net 4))
 (segment (start 223.21 71.56) (end 221.02 73.75) (width 0.25) (layer "B.Cu") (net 4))
 (segment (start 232.48 119.05) (end 236.29 119.05) (width 0.25) (layer "B.Cu") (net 4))
 (segment (start 255.34 122.86) (end 257.88 125.4) (width 0.25) (layer "B.Cu") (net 4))
 (segment (start 257.02 72.56) (end 256.02 71.56) (width 0.25) (layer "B.Cu") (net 4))
 (segment (start 235.02 93.249775) (end 235.02 91.618) (width 0.25) (layer "B.Cu") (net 4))
 (segment (start 239.02 73.94) (end 236.64 71.56) (width 0.25) (layer "B.Cu") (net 4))
 (segment (start 252.8 122.86) (end 252.8 108.489775) (width 0.25) (layer "B.Cu") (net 23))
 (segment (start 255.34 125.4) (end 252.8 122.86) (width 0.25) (layer "B.Cu") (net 23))
 (segment (start 250.26 122.86) (end 255.34 127.94) (width 0.25) (layer "B.Cu") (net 22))
 (segment (start 250.26 108.489775) (end 250.26 122.86) (width 0.25) (layer "B.Cu") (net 22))
 (segment (start 247.72 122.86) (end 255.34 130.48) (width 0.25) (layer "B.Cu") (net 21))
 (segment (start 247.72 108.489775) (end 247.72 122.86) (width 0.25) (layer "B.Cu") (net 21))
 (segment (start 227.4 108.489775) (end 227.4 112.7) (width 0.25) (layer "B.Cu") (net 17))
 (segment (start 235.02 115.24) (end 237.56 112.7) (width 0.25) (layer "F.Cu") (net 18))
 (segment (start 233.75 126.67) (end 235.02 125.4) (width 0.25) (layer "F.Cu") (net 18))
 (segment (start 235.02 125.4) (end 235.02 115.24) (width 0.25) (layer "F.Cu") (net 18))
 (segment (start 232.48 126.67) (end 233.75 126.67) (width 0.25) (layer "F.Cu") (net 18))
 (segment (start 210.74 132.73) (end 217.24 132.73) (width 0.25) (layer "B.Cu") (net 18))
 (segment (start 223.3 126.67) (end 217.24 132.73) (width 0.25) (layer "B.Cu") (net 18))
 (segment (start 234.150225 112.7) (end 237.56 112.7) (width 0.25) (layer "B.Cu") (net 18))
 (segment (start 229.94 112.7) (end 237.56 112.7) (width 0.25) (layer "B.Cu") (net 18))
 (segment (start 232.48 126.67) (end 223.3 126.67) (width 0.25) (layer "B.Cu") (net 18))
 (segment (start 229.94 108.489775) (end 234.150225 112.7) (width 0.25) (layer "B.Cu") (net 18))
 (segment (start 245.18 122.86) (end 245.18 108.489775) (width 0.25) (layer "B.Cu") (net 11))
 (segment (start 242.64 122.86) (end 242.64 108.489775) (width 0.25) (layer "B.Cu") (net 12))
 (segment (start 257.88 112.7) (end 257.88 108.489775) (width 0.25) (layer "B.Cu") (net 6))
 (segment (start 235.02 79.81) (end 237.27 79.81) (width 0.25) (layer "B.Cu") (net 5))
 (segment (start 237.27 79.81) (end 239.02 81.56) (width 0.25) (layer "B.Cu") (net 5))
 (segment (start 239.02 81.56) (end 243.650225 81.56) (width 0.25) (layer "B.Cu") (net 5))
 (segment (start 243.650225 81.56) (end 255.34 93.249775) (width 0.25) (layer "B.Cu") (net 5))
 (segment (start 235.02 79.81) (end 228.52 79.81) (width 0.25) (layer "B.Cu") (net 5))
 (segment (start 221.02 81.37) (end 222.335 82.685) (width 0.25) (layer "B.Cu") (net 7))
 (segment (start 216.27 79.81) (end 209.77 79.81) (width 0.25) (layer "B.Cu") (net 7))
 (segment (start 242.235225 82.685) (end 252.8 93.249775) (width 0.25) (layer "B.Cu") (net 7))
 (segment (start 217.83 81.37) (end 221.02 81.37) (width 0.25) (layer "B.Cu") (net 7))
 (segment (start 222.335 82.685) (end 242.235225 82.685) (width 0.25) (layer "B.Cu") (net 7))
 (segment (start 216.27 79.81) (end 217.83 81.37) (width 0.25) (layer "B.Cu") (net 7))
 (segment (start 253.02 79.81) (end 246.52 79.81) (width 0.25) (layer "B.Cu") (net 3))
 (segment (start 257.02 92.389775) (end 257.88 93.249775) (width 0.25) (layer "B.Cu") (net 3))
 (segment (start 257.02 81.37) (end 257.02 92.389775) (width 0.25) (layer "B.Cu") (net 3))
 (segment (start 253.02 79.81) (end 254.58 81.37) (width 0.25) (layer "B.Cu") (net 3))
 (segment (start 254.58 81.37) (end 257.02 81.37) (width 0.25) (layer "B.Cu") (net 3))
 (segment (start 224.86 108.489775) (end 224.86 112.7) (width 0.25) (layer "B.Cu") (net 8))
 (segment (start 202 112.7) (end 212.16 122.86) (width 0.25) (layer "B.Cu") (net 8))
 (segment (start 219.78 122.86) (end 224.86 117.78) (width 0.25) (layer "B.Cu") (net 8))
 (segment (start 224.86 112.7) (end 224.86 117.78) (width 0.25) (layer "B.Cu") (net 8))
 (segment (start 212.16 122.86) (end 219.78 122.86) (width 0.25) (layer "B.Cu") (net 8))
 (segment (start 222.32 108.489775) (end 222.32 112.7) (width 0.25) (layer "B.Cu") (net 9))
 (segment (start 202.545225 109.614775) (end 203.994775 109.614775) (width 0.25) (layer "B.Cu") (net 9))
 (segment (start 202 110.16) (end 202.545225 109.614775) (width 0.25) (layer "B.Cu") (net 9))
 (segment (start 222.32 112.7) (end 222.32 117.78) (width 0.25) (layer "B.Cu") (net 9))
 (segment (start 214.7 120.32) (end 219.78 120.32) (width 0.25) (layer "B.Cu") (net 9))
 (segment (start 203.994775 109.614775) (end 214.7 120.32) (width 0.25) (layer "B.Cu") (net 9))
 (segment (start 219.78 120.32) (end 222.32 117.78) (width 0.25) (layer "B.Cu") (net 9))
 (segment (start 202 92.38) (end 204.54 94.92) (width 0.25) (layer "B.Cu") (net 10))
 (segment (start 204.54 100.869775) (end 212.16 108.489775) (width 0.25) (layer "B.Cu") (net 10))
 (segment (start 204.54 94.92) (end 204.54 100.869775) (width 0.25) (layer "B.Cu") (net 10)))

